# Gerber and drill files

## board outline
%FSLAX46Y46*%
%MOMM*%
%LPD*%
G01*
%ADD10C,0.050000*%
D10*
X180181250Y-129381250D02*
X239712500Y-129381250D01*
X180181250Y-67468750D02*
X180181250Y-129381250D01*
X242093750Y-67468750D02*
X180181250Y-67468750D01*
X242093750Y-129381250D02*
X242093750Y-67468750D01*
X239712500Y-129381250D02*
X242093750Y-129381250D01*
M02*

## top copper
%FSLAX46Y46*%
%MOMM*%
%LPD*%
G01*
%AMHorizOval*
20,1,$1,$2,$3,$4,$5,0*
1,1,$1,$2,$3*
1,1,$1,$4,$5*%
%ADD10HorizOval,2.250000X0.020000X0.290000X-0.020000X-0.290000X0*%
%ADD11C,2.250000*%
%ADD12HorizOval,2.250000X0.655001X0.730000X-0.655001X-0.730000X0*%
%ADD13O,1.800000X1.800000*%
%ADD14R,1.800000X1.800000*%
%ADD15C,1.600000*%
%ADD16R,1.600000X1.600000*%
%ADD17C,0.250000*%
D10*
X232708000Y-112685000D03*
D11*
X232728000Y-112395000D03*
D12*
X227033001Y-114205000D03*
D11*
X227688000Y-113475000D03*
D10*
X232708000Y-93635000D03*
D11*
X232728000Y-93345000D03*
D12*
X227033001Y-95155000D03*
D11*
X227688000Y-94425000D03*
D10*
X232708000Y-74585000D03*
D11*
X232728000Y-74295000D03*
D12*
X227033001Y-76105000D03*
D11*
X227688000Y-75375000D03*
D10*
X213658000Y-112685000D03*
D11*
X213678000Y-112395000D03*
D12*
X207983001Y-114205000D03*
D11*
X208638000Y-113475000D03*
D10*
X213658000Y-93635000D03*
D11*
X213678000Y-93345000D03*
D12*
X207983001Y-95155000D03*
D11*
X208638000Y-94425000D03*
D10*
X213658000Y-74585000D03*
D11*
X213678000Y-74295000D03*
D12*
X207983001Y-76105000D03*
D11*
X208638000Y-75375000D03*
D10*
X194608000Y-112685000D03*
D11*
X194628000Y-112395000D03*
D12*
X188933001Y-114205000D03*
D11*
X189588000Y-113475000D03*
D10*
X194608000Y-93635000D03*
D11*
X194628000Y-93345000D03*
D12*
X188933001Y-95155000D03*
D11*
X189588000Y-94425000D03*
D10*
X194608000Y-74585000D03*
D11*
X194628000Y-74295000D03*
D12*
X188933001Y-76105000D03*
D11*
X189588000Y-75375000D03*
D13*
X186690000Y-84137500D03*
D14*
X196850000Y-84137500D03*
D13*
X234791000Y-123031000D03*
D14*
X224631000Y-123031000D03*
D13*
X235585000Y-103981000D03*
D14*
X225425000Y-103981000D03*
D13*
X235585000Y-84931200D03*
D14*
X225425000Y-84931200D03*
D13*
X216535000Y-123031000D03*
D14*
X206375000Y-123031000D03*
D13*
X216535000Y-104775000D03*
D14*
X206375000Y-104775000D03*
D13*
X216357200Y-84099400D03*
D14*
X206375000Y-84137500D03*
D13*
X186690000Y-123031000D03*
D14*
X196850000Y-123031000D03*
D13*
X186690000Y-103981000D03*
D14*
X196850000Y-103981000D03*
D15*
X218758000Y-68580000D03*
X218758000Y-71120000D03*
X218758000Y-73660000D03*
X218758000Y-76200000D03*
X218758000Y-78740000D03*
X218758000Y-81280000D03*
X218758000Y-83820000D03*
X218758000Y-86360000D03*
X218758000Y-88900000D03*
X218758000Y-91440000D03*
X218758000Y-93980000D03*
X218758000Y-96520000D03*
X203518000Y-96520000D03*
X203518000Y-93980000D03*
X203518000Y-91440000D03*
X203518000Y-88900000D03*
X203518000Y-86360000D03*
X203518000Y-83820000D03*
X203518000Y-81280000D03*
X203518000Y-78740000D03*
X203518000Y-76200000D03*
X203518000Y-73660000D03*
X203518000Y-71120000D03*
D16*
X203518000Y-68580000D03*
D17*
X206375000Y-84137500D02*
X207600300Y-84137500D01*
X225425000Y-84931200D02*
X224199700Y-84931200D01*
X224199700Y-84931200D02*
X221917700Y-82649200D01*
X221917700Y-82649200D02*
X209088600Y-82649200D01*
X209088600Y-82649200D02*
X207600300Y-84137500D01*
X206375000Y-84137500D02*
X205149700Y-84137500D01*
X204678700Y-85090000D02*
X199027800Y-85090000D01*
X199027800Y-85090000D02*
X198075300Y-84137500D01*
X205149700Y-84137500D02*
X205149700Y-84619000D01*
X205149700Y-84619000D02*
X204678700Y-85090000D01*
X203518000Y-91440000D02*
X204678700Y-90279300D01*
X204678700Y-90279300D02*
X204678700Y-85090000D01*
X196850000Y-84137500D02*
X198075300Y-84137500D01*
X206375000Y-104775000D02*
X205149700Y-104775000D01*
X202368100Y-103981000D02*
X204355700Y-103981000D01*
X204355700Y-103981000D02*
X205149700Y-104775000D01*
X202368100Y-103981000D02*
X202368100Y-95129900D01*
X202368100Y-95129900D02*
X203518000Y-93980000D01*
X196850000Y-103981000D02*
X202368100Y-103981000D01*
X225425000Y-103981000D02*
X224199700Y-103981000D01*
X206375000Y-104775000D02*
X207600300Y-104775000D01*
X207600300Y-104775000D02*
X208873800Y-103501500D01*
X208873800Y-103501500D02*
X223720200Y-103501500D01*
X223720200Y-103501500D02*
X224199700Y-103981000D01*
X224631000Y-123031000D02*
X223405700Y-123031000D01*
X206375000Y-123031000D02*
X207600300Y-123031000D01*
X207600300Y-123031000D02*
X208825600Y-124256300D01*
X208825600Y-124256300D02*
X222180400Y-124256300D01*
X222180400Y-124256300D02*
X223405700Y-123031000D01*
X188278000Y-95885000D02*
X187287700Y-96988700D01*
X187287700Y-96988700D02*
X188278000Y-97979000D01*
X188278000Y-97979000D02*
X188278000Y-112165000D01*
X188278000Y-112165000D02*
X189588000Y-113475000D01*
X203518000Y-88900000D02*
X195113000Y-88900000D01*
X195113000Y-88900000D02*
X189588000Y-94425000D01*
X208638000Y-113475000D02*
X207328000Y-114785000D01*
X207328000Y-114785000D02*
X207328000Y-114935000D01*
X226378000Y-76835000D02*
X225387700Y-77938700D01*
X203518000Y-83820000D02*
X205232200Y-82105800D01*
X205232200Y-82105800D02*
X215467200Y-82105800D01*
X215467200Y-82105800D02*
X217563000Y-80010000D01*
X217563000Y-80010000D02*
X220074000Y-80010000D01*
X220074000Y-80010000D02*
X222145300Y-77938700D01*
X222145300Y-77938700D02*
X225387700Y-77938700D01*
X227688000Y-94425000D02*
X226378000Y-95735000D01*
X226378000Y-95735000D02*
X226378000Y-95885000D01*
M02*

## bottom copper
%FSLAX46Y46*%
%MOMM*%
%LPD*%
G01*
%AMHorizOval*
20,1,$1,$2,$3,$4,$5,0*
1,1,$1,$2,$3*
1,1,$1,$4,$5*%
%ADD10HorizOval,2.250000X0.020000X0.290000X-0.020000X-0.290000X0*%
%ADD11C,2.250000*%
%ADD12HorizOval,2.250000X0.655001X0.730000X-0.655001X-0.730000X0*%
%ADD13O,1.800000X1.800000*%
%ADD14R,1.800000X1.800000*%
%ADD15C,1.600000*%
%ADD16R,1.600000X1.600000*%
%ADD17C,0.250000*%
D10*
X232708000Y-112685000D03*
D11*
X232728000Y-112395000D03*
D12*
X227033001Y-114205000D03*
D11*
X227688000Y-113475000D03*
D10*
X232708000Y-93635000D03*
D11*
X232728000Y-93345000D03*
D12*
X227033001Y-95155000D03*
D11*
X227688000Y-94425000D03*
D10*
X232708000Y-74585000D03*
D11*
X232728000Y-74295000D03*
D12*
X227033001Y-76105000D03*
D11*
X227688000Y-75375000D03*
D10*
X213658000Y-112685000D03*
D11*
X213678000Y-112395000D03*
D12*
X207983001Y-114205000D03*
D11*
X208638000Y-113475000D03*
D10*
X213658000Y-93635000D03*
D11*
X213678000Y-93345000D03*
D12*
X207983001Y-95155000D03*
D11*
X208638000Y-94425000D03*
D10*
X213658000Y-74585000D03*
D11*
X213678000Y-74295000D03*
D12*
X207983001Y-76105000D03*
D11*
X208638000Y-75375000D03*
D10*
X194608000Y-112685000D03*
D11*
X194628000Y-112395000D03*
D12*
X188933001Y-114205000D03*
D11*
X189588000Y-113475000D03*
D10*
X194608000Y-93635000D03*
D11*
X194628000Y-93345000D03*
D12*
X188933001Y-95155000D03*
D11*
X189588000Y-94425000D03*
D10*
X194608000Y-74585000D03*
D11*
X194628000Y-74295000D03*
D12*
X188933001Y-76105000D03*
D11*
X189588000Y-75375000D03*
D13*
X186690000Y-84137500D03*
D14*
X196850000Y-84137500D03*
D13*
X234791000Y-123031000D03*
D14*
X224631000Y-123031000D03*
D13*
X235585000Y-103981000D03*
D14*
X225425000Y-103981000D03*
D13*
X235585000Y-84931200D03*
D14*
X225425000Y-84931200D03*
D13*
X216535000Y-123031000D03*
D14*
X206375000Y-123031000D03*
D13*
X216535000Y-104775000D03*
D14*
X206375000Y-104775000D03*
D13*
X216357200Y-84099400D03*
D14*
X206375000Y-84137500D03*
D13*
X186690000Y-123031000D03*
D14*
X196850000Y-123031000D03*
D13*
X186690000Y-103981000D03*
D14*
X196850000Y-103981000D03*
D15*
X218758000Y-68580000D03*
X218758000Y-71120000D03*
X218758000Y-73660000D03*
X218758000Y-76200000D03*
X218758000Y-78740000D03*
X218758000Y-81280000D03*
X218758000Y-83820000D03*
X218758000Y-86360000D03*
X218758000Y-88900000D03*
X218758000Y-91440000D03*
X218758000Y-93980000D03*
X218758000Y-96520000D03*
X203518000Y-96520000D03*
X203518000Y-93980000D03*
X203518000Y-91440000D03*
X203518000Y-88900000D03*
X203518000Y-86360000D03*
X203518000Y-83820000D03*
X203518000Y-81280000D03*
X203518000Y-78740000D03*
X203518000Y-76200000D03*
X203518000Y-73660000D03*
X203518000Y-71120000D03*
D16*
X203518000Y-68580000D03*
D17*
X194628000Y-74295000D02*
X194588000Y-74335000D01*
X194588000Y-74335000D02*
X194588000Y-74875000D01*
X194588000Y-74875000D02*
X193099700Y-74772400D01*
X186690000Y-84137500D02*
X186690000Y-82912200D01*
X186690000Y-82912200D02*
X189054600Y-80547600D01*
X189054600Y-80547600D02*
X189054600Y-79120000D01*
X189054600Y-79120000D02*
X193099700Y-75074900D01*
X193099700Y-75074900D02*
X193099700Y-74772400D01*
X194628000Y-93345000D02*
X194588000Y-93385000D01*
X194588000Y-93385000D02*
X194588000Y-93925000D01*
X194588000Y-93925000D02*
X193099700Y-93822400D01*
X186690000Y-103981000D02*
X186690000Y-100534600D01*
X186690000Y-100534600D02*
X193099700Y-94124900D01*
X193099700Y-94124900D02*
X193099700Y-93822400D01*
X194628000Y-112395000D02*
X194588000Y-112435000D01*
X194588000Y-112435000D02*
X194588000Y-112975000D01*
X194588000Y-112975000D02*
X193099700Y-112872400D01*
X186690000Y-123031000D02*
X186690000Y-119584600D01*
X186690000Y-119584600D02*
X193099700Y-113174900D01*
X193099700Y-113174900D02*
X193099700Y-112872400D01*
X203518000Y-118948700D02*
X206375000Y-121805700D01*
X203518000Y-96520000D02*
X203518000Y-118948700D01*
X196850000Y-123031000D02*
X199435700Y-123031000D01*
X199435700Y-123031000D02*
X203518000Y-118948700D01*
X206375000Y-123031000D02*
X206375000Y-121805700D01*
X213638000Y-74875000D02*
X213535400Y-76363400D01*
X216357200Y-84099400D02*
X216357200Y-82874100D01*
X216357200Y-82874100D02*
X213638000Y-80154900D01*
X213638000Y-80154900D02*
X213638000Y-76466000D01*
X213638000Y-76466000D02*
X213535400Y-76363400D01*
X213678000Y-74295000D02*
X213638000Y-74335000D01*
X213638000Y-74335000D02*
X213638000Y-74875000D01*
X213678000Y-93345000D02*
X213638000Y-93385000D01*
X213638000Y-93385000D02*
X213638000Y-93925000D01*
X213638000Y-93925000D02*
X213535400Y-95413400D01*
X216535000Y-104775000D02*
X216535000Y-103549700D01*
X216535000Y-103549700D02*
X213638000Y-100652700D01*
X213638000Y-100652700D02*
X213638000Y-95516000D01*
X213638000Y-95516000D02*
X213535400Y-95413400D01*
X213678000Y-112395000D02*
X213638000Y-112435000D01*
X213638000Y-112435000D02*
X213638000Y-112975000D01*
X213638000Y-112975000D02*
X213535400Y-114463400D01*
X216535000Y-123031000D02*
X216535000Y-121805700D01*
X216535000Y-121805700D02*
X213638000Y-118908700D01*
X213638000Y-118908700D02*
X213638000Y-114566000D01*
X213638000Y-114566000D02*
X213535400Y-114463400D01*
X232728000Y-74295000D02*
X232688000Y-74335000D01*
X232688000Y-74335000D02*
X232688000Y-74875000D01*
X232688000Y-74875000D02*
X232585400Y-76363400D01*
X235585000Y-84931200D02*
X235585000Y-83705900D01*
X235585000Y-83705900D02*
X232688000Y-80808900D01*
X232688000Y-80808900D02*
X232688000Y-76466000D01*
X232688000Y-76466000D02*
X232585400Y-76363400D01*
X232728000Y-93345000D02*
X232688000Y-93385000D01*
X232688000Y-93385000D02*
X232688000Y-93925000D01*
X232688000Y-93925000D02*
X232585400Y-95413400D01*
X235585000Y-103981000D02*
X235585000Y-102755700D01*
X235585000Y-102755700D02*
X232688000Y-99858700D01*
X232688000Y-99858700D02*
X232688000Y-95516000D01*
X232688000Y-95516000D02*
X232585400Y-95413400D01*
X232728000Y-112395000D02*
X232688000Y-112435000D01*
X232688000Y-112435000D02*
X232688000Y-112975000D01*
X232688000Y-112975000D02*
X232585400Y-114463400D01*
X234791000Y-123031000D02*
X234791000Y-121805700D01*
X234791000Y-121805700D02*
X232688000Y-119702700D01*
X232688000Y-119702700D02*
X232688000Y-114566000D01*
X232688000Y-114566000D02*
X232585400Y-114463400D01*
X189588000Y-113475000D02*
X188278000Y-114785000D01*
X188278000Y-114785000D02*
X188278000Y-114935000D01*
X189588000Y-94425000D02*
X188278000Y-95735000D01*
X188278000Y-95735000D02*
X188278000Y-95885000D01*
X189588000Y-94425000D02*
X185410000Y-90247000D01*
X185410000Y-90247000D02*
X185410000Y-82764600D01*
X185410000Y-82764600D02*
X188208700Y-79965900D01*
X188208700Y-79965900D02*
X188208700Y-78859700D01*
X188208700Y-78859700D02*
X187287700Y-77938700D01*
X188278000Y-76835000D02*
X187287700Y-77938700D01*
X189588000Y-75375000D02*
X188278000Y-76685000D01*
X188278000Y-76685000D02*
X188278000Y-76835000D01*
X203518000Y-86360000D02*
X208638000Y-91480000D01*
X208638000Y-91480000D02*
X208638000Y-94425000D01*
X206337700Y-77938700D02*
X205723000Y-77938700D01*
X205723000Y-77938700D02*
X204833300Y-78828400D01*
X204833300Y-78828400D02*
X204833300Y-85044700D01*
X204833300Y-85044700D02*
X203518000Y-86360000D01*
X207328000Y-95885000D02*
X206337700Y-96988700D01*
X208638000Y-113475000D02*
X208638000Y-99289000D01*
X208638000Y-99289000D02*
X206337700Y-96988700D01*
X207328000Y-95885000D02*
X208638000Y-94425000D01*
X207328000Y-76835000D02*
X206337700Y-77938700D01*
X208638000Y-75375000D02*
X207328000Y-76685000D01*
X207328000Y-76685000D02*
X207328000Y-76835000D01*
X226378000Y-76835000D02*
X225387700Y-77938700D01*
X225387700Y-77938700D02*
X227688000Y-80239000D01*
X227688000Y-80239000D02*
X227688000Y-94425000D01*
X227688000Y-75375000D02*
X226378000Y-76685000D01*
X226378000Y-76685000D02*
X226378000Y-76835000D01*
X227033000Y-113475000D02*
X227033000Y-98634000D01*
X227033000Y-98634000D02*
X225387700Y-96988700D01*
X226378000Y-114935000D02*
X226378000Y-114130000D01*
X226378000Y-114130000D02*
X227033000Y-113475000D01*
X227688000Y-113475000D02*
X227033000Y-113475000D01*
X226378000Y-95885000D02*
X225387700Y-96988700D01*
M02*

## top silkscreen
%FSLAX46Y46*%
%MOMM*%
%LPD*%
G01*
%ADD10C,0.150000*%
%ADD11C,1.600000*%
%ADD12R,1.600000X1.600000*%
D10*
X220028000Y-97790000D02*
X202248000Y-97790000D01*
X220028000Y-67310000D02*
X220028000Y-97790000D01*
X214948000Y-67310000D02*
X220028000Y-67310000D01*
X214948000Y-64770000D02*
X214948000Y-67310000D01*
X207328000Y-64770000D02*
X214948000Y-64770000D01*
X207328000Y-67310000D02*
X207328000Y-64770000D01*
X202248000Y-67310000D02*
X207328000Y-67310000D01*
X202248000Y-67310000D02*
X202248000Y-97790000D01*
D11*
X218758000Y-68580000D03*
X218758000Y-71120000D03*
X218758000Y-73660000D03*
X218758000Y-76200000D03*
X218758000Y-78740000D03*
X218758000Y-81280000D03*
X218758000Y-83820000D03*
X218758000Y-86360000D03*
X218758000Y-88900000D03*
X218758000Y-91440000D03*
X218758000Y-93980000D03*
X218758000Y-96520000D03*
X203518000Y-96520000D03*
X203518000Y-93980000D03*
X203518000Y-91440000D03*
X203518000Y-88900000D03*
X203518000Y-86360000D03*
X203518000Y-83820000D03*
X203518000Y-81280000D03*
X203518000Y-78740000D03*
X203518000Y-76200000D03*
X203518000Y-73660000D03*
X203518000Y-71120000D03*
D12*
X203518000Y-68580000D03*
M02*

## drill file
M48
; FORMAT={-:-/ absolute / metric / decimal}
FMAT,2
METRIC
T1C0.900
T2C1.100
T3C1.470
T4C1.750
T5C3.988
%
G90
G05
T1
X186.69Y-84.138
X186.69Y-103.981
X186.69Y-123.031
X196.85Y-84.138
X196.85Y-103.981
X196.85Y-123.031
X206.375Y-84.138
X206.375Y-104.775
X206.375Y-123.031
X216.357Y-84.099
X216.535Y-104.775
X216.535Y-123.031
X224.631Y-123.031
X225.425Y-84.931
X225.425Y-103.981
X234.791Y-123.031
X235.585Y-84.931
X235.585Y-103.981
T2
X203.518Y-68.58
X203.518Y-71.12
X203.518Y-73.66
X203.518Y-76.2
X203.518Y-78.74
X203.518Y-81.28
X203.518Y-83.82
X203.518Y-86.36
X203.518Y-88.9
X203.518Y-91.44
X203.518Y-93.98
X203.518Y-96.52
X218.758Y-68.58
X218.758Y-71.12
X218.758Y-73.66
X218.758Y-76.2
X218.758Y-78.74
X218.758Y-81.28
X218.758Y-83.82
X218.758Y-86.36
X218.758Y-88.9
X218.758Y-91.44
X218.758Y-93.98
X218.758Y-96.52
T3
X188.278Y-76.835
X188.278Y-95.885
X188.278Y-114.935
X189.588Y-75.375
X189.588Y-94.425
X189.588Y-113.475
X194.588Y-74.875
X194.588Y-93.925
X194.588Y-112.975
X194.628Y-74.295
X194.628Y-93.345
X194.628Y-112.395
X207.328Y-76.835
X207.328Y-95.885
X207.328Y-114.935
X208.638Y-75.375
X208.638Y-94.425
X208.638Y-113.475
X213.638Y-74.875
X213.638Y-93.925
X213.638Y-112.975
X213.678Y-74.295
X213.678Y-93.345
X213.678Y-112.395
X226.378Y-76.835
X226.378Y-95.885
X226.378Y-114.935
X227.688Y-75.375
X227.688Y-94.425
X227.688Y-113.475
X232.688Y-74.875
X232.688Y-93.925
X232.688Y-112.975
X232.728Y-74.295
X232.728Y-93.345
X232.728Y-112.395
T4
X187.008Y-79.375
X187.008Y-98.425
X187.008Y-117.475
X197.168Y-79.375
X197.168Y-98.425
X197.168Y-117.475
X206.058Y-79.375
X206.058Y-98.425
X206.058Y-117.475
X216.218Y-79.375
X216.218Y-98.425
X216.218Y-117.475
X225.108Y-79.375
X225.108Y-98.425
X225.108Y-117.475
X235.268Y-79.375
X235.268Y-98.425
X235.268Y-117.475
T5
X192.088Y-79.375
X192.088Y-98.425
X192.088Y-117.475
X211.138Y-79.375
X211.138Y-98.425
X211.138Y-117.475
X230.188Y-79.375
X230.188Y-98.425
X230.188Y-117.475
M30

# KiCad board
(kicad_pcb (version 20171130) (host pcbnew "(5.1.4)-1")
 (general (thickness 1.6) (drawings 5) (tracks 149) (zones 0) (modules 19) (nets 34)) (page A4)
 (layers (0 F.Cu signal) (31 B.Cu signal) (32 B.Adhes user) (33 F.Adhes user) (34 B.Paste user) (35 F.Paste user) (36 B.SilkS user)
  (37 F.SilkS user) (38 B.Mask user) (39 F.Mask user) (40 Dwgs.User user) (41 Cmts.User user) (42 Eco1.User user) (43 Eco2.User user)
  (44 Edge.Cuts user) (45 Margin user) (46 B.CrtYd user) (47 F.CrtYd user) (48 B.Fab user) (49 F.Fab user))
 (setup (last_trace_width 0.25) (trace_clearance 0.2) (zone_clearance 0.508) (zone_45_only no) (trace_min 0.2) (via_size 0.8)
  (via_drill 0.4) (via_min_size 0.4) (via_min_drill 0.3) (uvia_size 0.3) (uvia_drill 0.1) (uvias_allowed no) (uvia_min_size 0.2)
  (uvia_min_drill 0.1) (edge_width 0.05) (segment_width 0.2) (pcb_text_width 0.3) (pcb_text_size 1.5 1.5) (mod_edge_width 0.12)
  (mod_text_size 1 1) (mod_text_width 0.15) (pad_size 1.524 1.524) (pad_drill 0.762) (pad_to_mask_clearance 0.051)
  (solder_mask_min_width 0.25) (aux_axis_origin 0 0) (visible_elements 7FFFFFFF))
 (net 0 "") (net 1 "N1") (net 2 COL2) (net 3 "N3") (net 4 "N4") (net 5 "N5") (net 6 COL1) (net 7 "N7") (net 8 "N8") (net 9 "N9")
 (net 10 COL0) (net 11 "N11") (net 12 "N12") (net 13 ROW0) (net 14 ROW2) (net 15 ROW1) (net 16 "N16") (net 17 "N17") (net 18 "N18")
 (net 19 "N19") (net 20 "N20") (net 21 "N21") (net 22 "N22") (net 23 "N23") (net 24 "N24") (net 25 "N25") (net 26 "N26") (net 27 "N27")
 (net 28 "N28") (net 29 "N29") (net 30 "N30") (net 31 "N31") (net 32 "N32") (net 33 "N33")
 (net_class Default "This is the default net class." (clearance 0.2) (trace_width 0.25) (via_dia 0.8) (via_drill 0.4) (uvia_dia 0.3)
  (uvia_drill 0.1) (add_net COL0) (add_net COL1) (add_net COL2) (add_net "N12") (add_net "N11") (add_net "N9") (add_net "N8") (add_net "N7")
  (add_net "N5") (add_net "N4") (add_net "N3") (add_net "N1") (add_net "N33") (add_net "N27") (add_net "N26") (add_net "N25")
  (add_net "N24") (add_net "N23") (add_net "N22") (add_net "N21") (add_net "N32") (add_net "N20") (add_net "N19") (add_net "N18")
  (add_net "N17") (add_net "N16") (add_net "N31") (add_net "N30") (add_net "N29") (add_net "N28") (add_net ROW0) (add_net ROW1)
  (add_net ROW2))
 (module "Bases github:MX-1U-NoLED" (layer F.Cu) (at 230.188 117.475)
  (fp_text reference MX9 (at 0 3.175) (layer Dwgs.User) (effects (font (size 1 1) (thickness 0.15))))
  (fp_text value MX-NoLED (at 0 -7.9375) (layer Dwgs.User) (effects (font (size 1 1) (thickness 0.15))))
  (pad 2 thru_hole oval (at 2.5 -4.5 86.0548) (size 2.831378 2.25) (drill 1.47 (offset 0.290689 0)) (layers *.Cu B.Mask) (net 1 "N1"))
  (pad 2 thru_hole circle (at 2.54 -5.08) (size 2.25 2.25) (drill 1.47) (layers *.Cu B.Mask) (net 1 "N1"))
  (pad 1 thru_hole oval (at -3.81 -2.54 48.0996) (size 4.211556 2.25) (drill 1.47 (offset 0.980778 0)) (layers *.Cu B.Mask) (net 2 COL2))
  (pad "" np_thru_hole circle (at 0 0) (size 3.9878 3.9878) (drill 3.9878) (layers *.Cu *.Mask))
  (pad 1 thru_hole circle (at -2.5 -4) (size 2.25 2.25) (drill 1.47) (layers *.Cu B.Mask) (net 2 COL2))
  (pad "" np_thru_hole circle (at -5.08 0 48.0996) (size 1.75 1.75) (drill 1.75) (layers *.Cu *.Mask))
  (pad "" np_thru_hole circle (at 5.08 0 48.0996) (size 1.75 1.75) (drill 1.75) (layers *.Cu *.Mask)))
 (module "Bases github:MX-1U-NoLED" (layer F.Cu) (at 230.188 98.425)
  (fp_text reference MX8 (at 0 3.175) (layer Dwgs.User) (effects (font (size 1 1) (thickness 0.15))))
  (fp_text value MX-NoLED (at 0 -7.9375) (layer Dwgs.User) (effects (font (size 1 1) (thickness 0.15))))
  (pad 2 thru_hole oval (at 2.5 -4.5 86.0548) (size 2.831378 2.25) (drill 1.47 (offset 0.290689 0)) (layers *.Cu B.Mask) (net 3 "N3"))
  (pad 2 thru_hole circle (at 2.54 -5.08) (size 2.25 2.25) (drill 1.47) (layers *.Cu B.Mask) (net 3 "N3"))
  (pad 1 thru_hole oval (at -3.81 -2.54 48.0996) (size 4.211556 2.25) (drill 1.47 (offset 0.980778 0)) (layers *.Cu B.Mask) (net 2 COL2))
  (pad "" np_thru_hole circle (at 0 0) (size 3.9878 3.9878) (drill 3.9878) (layers *.Cu *.Mask))
  (pad 1 thru_hole circle (at -2.5 -4) (size 2.25 2.25) (drill 1.47) (layers *.Cu B.Mask) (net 2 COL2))
  (pad "" np_thru_hole circle (at -5.08 0 48.0996) (size 1.75 1.75) (drill 1.75) (layers *.Cu *.Mask))
  (pad "" np_thru_hole circle (at 5.08 0 48.0996) (size 1.75 1.75) (drill 1.75) (layers *.Cu *.Mask)))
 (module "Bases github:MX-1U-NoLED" (layer F.Cu) (at 230.188 79.375)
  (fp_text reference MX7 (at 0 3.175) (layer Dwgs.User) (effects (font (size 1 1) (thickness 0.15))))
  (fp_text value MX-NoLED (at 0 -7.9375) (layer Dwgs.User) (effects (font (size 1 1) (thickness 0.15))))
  (pad 2 thru_hole oval (at 2.5 -4.5 86.0548) (size 2.831378 2.25) (drill 1.47 (offset 0.290689 0)) (layers *.Cu B.Mask) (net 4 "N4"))
  (pad 2 thru_hole circle (at 2.54 -5.08) (size 2.25 2.25) (drill 1.47) (layers *.Cu B.Mask) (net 4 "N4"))
  (pad 1 thru_hole oval (at -3.81 -2.54 48.0996) (size 4.211556 2.25) (drill 1.47 (offset 0.980778 0)) (layers *.Cu B.Mask) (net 2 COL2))
  (pad "" np_thru_hole circle (at 0 0) (size 3.9878 3.9878) (drill 3.9878) (layers *.Cu *.Mask))
  (pad 1 thru_hole circle (at -2.5 -4) (size 2.25 2.25) (drill 1.47) (layers *.Cu B.Mask) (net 2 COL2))
  (pad "" np_thru_hole circle (at -5.08 0 48.0996) (size 1.75 1.75) (drill 1.75) (layers *.Cu *.Mask))
  (pad "" np_thru_hole circle (at 5.08 0 48.0996) (size 1.75 1.75) (drill 1.75) (layers *.Cu *.Mask)))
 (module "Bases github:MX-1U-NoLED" (layer F.Cu) (at 211.138 117.475)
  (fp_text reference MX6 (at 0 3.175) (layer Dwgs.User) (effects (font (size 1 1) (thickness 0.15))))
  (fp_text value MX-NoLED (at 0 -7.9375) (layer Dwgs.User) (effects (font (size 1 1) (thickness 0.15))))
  (pad 2 thru_hole oval (at 2.5 -4.5 86.0548) (size 2.831378 2.25) (drill 1.47 (offset 0.290689 0)) (layers *.Cu B.Mask) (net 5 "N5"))
  (pad 2 thru_hole circle (at 2.54 -5.08) (size 2.25 2.25) (drill 1.47) (layers *.Cu B.Mask) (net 5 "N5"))
  (pad 1 thru_hole oval (at -3.81 -2.54 48.0996) (size 4.211556 2.25) (drill 1.47 (offset 0.980778 0)) (layers *.Cu B.Mask) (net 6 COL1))
  (pad "" np_thru_hole circle (at 0 0) (size 3.9878 3.9878) (drill 3.9878) (layers *.Cu *.Mask))
  (pad 1 thru_hole circle (at -2.5 -4) (size 2.25 2.25) (drill 1.47) (layers *.Cu B.Mask) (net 6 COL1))
  (pad "" np_thru_hole circle (at -5.08 0 48.0996) (size 1.75 1.75) (drill 1.75) (layers *.Cu *.Mask))
  (pad "" np_thru_hole circle (at 5.08 0 48.0996) (size 1.75 1.75) (drill 1.75) (layers *.Cu *.Mask)))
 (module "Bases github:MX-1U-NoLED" (layer F.Cu) (at 211.138 98.425)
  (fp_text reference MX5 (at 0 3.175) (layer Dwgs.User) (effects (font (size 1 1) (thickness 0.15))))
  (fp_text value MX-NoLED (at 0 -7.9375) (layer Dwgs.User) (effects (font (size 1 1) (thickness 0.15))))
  (pad 2 thru_hole oval (at 2.5 -4.5 86.0548) (size 2.831378 2.25) (drill 1.47 (offset 0.290689 0)) (layers *.Cu B.Mask) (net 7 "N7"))
  (pad 2 thru_hole circle (at 2.54 -5.08) (size 2.25 2.25) (drill 1.47) (layers *.Cu B.Mask) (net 7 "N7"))
  (pad 1 thru_hole oval (at -3.81 -2.54 48.0996) (size 4.211556 2.25) (drill 1.47 (offset 0.980778 0)) (layers *.Cu B.Mask) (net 6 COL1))
  (pad "" np_thru_hole circle (at 0 0) (size 3.9878 3.9878) (drill 3.9878) (layers *.Cu *.Mask))
  (pad 1 thru_hole circle (at -2.5 -4) (size 2.25 2.25) (drill 1.47) (layers *.Cu B.Mask) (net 6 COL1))
  (pad "" np_thru_hole circle (at -5.08 0 48.0996) (size 1.75 1.75) (drill 1.75) (layers *.Cu *.Mask))
  (pad "" np_thru_hole circle (at 5.08 0 48.0996) (size 1.75 1.75) (drill 1.75) (layers *.Cu *.Mask)))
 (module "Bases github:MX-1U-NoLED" (layer F.Cu) (at 211.138 79.375)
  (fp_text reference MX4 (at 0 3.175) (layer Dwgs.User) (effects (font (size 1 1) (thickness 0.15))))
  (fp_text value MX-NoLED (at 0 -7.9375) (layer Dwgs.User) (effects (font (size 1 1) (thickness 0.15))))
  (pad 2 thru_hole oval (at 2.5 -4.5 86.0548) (size 2.831378 2.25) (drill 1.47 (offset 0.290689 0)) (layers *.Cu B.Mask) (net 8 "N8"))
  (pad 2 thru_hole circle (at 2.54 -5.08) (size 2.25 2.25) (drill 1.47) (layers *.Cu B.Mask) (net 8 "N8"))
  (pad 1 thru_hole oval (at -3.81 -2.54 48.0996) (size 4.211556 2.25) (drill 1.47 (offset 0.980778 0)) (layers *.Cu B.Mask) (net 6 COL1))
  (pad "" np_thru_hole circle (at 0 0) (size 3.9878 3.9878) (drill 3.9878) (layers *.Cu *.Mask))
  (pad 1 thru_hole circle (at -2.5 -4) (size 2.25 2.25) (drill 1.47) (layers *.Cu B.Mask) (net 6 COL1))
  (pad "" np_thru_hole circle (at -5.08 0 48.0996) (size 1.75 1.75) (drill 1.75) (layers *.Cu *.Mask))
  (pad "" np_thru_hole circle (at 5.08 0 48.0996) (size 1.75 1.75) (drill 1.75) (layers *.Cu *.Mask)))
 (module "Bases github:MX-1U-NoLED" (layer F.Cu) (at 192.088 117.475)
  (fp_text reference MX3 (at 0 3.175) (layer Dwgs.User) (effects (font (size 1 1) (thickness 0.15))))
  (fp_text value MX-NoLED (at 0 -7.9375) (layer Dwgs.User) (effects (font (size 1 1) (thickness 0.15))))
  (pad 2 thru_hole oval (at 2.5 -4.5 86.0548) (size 2.831378 2.25) (drill 1.47 (offset 0.290689 0)) (layers *.Cu B.Mask) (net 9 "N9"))
  (pad 2 thru_hole circle (at 2.54 -5.08) (size 2.25 2.25) (drill 1.47) (layers *.Cu B.Mask) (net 9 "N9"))
  (pad 1 thru_hole oval (at -3.81 -2.54 48.0996) (size 4.211556 2.25) (drill 1.47 (offset 0.980778 0)) (layers *.Cu B.Mask) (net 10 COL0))
  (pad "" np_thru_hole circle (at 0 0) (size 3.9878 3.9878) (drill 3.9878) (layers *.Cu *.Mask))
  (pad 1 thru_hole circle (at -2.5 -4) (size 2.25 2.25) (drill 1.47) (layers *.Cu B.Mask) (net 10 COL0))
  (pad "" np_thru_hole circle (at -5.08 0 48.0996) (size 1.75 1.75) (drill 1.75) (layers *.Cu *.Mask))
  (pad "" np_thru_hole circle (at 5.08 0 48.0996) (size 1.75 1.75) (drill 1.75) (layers *.Cu *.Mask)))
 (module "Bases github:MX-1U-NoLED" (layer F.Cu) (at 192.088 98.425)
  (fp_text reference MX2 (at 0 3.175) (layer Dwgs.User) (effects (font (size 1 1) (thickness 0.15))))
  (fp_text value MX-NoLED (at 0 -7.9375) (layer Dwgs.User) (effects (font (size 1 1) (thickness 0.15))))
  (pad 2 thru_hole oval (at 2.5 -4.5 86.0548) (size 2.831378 2.25) (drill 1.47 (offset 0.290689 0)) (layers *.Cu B.Mask) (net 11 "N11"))
  (pad 2 thru_hole circle (at 2.54 -5.08) (size 2.25 2.25) (drill 1.47) (layers *.Cu B.Mask) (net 11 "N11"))
  (pad 1 thru_hole oval (at -3.81 -2.54 48.0996) (size 4.211556 2.25) (drill 1.47 (offset 0.980778 0)) (layers *.Cu B.Mask) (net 10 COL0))
  (pad "" np_thru_hole circle (at 0 0) (size 3.9878 3.9878) (drill 3.9878) (layers *.Cu *.Mask))
  (pad 1 thru_hole circle (at -2.5 -4) (size 2.25 2.25) (drill 1.47) (layers *.Cu B.Mask) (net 10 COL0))
  (pad "" np_thru_hole circle (at -5.08 0 48.0996) (size 1.75 1.75) (drill 1.75) (layers *.Cu *.Mask))
  (pad "" np_thru_hole circle (at 5.08 0 48.0996) (size 1.75 1.75) (drill 1.75) (layers *.Cu *.Mask)))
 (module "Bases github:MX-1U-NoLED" (layer F.Cu) (at 192.088 79.375)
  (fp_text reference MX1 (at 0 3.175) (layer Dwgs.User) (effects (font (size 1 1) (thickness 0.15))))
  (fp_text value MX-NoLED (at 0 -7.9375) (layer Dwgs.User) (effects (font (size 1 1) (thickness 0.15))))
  (pad 2 thru_hole oval (at 2.5 -4.5 86.0548) (size 2.831378 2.25) (drill 1.47 (offset 0.290689 0)) (layers *.Cu B.Mask) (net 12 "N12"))
  (pad 2 thru_hole circle (at 2.54 -5.08) (size 2.25 2.25) (drill 1.47) (layers *.Cu B.Mask) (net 12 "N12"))
  (pad 1 thru_hole oval (at -3.81 -2.54 48.0996) (size 4.211556 2.25) (drill 1.47 (offset 0.980778 0)) (layers *.Cu B.Mask) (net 10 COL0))
  (pad "" np_thru_hole circle (at 0 0) (size 3.9878 3.9878) (drill 3.9878) (layers *.Cu *.Mask))
  (pad 1 thru_hole circle (at -2.5 -4) (size 2.25 2.25) (drill 1.47) (layers *.Cu B.Mask) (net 10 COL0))
  (pad "" np_thru_hole circle (at -5.08 0 48.0996) (size 1.75 1.75) (drill 1.75) (layers *.Cu *.Mask))
  (pad "" np_thru_hole circle (at 5.08 0 48.0996) (size 1.75 1.75) (drill 1.75) (layers *.Cu *.Mask)))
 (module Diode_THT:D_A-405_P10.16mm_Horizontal (layer B.Cu) (at 196.85 84.1375 180)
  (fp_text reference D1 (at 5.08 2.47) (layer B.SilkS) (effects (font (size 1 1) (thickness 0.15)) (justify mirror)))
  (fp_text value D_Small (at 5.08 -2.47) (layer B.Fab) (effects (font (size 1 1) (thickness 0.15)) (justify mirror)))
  (pad 2 thru_hole oval (at 10.16 0 180) (size 1.8 1.8) (drill 0.9) (layers *.Cu *.Mask) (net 12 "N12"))
  (pad 1 thru_hole rect (at 0 0 180) (size 1.8 1.8) (drill 0.9) (layers *.Cu *.Mask) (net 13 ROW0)))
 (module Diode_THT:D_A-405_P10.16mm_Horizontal (layer B.Cu) (at 224.631 123.031)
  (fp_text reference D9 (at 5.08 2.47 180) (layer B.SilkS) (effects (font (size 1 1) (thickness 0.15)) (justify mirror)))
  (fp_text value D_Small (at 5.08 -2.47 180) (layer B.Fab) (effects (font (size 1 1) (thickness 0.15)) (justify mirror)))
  (pad 2 thru_hole oval (at 10.16 0) (size 1.8 1.8) (drill 0.9) (layers *.Cu *.Mask) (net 1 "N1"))
  (pad 1 thru_hole rect (at 0 0) (size 1.8 1.8) (drill 0.9) (layers *.Cu *.Mask) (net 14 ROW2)))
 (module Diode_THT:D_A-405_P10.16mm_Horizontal (layer B.Cu) (at 225.425 103.981)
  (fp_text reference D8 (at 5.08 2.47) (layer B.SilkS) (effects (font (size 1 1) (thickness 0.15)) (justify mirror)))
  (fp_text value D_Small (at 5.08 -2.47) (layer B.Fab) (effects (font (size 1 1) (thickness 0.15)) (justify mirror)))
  (pad 2 thru_hole oval (at 10.16 0) (size 1.8 1.8) (drill 0.9) (layers *.Cu *.Mask) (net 3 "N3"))
  (pad 1 thru_hole rect (at 0 0) (size 1.8 1.8) (drill 0.9) (layers *.Cu *.Mask) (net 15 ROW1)))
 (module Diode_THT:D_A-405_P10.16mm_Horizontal (layer B.Cu) (at 225.425 84.9312)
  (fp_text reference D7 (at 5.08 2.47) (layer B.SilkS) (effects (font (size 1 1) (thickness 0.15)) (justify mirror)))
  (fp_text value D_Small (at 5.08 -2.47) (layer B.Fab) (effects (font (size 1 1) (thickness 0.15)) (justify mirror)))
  (pad 2 thru_hole oval (at 10.16 0) (size 1.8 1.8) (drill 0.9) (layers *.Cu *.Mask) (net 4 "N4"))
  (pad 1 thru_hole rect (at 0 0) (size 1.8 1.8) (drill 0.9) (layers *.Cu *.Mask) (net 13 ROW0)))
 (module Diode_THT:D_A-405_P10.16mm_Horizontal (layer B.Cu) (at 206.375 123.031)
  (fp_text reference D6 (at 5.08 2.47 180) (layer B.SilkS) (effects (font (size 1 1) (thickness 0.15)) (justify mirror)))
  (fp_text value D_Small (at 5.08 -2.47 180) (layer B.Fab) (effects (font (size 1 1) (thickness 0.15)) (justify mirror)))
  (pad 2 thru_hole oval (at 10.16 0) (size 1.8 1.8) (drill 0.9) (layers *.Cu *.Mask) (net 5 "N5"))
  (pad 1 thru_hole rect (at 0 0) (size 1.8 1.8) (drill 0.9) (layers *.Cu *.Mask) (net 14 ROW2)))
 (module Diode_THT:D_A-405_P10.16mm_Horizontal (layer B.Cu) (at 206.375 104.775)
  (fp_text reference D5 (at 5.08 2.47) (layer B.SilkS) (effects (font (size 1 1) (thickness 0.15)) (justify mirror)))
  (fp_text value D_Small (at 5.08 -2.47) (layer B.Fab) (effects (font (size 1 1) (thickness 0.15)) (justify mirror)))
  (pad 2 thru_hole oval (at 10.16 0) (size 1.8 1.8) (drill 0.9) (layers *.Cu *.Mask) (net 7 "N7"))
  (pad 1 thru_hole rect (at 0 0) (size 1.8 1.8) (drill 0.9) (layers *.Cu *.Mask) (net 15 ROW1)))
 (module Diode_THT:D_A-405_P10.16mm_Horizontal (layer B.Cu) (at 206.375 84.1375)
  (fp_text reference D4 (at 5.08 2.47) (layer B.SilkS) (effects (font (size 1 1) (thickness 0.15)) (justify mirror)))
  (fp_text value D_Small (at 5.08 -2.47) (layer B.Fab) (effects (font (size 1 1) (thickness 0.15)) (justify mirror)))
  (pad 2 thru_hole oval (at 9.9822 -0.0381) (size 1.8 1.8) (drill 0.9) (layers *.Cu *.Mask) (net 8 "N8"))
  (pad 1 thru_hole rect (at 0 0) (size 1.8 1.8) (drill 0.9) (layers *.Cu *.Mask) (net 13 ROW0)))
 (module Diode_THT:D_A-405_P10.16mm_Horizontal (layer B.Cu) (at 196.85 123.031 180)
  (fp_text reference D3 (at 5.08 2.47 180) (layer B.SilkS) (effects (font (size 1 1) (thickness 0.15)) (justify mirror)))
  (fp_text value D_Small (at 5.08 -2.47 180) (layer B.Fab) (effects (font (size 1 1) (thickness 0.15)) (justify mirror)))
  (pad 2 thru_hole oval (at 10.16 0 180) (size 1.8 1.8) (drill 0.9) (layers *.Cu *.Mask) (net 9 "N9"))
  (pad 1 thru_hole rect (at 0 0 180) (size 1.8 1.8) (drill 0.9) (layers *.Cu *.Mask) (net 14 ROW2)))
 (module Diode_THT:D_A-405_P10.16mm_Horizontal (layer B.Cu) (at 196.85 103.981 180)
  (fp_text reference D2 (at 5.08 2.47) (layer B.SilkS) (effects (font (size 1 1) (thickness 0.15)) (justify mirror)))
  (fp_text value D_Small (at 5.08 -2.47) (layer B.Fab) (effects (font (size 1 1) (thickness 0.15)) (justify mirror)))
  (pad 2 thru_hole oval (at 10.16 0 180) (size 1.8 1.8) (drill 0.9) (layers *.Cu *.Mask) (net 11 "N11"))
  (pad 1 thru_hole rect (at 0 0 180) (size 1.8 1.8) (drill 0.9) (layers *.Cu *.Mask) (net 15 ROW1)))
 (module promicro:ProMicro (layer F.Cu) (at 211.138 82.55 270)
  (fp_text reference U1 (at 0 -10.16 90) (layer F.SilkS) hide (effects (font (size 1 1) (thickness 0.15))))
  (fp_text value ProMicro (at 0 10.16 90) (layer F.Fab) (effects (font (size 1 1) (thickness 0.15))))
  (fp_line (start 15.24 -8.89) (end 15.24 8.89) (layer F.SilkS) (width 0.15))
  (fp_line (start -15.24 -8.89) (end 15.24 -8.89) (layer F.SilkS) (width 0.15))
  (fp_line (start -15.24 -3.81) (end -15.24 -8.89) (layer F.SilkS) (width 0.15))
  (fp_line (start -17.78 -3.81) (end -15.24 -3.81) (layer F.SilkS) (width 0.15))
  (fp_line (start -17.78 3.81) (end -17.78 -3.81) (layer F.SilkS) (width 0.15))
  (fp_line (start -15.24 3.81) (end -17.78 3.81) (layer F.SilkS) (width 0.15))
  (fp_line (start -15.24 8.89) (end -15.24 3.81) (layer F.SilkS) (width 0.15))
  (fp_line (start -15.24 8.89) (end 15.24 8.89) (layer F.SilkS) (width 0.15))
  (pad 24 thru_hole circle (at -13.97 -7.62 270) (size 1.6 1.6) (drill 1.1) (layers *.Cu *.Mask F.SilkS) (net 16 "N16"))
  (pad 23 thru_hole circle (at -11.43 -7.62 270) (size 1.6 1.6) (drill 1.1) (layers *.Cu *.Mask F.SilkS) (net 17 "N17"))
  (pad 22 thru_hole circle (at -8.89 -7.62 270) (size 1.6 1.6) (drill 1.1) (layers *.Cu *.Mask F.SilkS) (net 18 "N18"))
  (pad 21 thru_hole circle (at -6.35 -7.62 270) (size 1.6 1.6) (drill 1.1) (layers *.Cu *.Mask F.SilkS) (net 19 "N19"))
  (pad 20 thru_hole circle (at -3.81 -7.62 270) (size 1.6 1.6) (drill 1.1) (layers *.Cu *.Mask F.SilkS) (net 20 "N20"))
  (pad 19 thru_hole circle (at -1.27 -7.62 270) (size 1.6 1.6) (drill 1.1) (layers *.Cu *.Mask F.SilkS) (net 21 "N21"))
  (pad 18 thru_hole circle (at 1.27 -7.62 270) (size 1.6 1.6) (drill 1.1) (layers *.Cu *.Mask F.SilkS) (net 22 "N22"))
  (pad 17 thru_hole circle (at 3.81 -7.62 270) (size 1.6 1.6) (drill 1.1) (layers *.Cu *.Mask F.SilkS) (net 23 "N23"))
  (pad 16 thru_hole circle (at 6.35 -7.62 270) (size 1.6 1.6) (drill 1.1) (layers *.Cu *.Mask F.SilkS) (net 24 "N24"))
  (pad 15 thru_hole circle (at 8.89 -7.62 270) (size 1.6 1.6) (drill 1.1) (layers *.Cu *.Mask F.SilkS) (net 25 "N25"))
  (pad 14 thru_hole circle (at 11.43 -7.62 270) (size 1.6 1.6) (drill 1.1) (layers *.Cu *.Mask F.SilkS) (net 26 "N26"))
  (pad 13 thru_hole circle (at 13.97 -7.62 270) (size 1.6 1.6) (drill 1.1) (layers *.Cu *.Mask F.SilkS) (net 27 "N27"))
  (pad 12 thru_hole circle (at 13.97 7.62 270) (size 1.6 1.6) (drill 1.1) (layers *.Cu *.Mask F.SilkS) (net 14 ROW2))
  (pad 11 thru_hole circle (at 11.43 7.62 270) (size 1.6 1.6) (drill 1.1) (layers *.Cu *.Mask F.SilkS) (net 15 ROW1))
  (pad 10 thru_hole circle (at 8.89 7.62 270) (size 1.6 1.6) (drill 1.1) (layers *.Cu *.Mask F.SilkS) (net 13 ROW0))
  (pad 9 thru_hole circle (at 6.35 7.62 270) (size 1.6 1.6) (drill 1.1) (layers *.Cu *.Mask F.SilkS) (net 10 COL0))
  (pad 8 thru_hole circle (at 3.81 7.62 270) (size 1.6 1.6) (drill 1.1) (layers *.Cu *.Mask F.SilkS) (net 6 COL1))
  (pad 7 thru_hole circle (at 1.27 7.62 270) (size 1.6 1.6) (drill 1.1) (layers *.Cu *.Mask F.SilkS) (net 2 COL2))
  (pad 6 thru_hole circle (at -1.27 7.62 270) (size 1.6 1.6) (drill 1.1) (layers *.Cu *.Mask F.SilkS) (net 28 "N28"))
  (pad 5 thru_hole circle (at -3.81 7.62 270) (size 1.6 1.6) (drill 1.1) (layers *.Cu *.Mask F.SilkS) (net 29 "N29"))
  (pad 4 thru_hole circle (at -6.35 7.62 270) (size 1.6 1.6) (drill 1.1) (layers *.Cu *.Mask F.SilkS) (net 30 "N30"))
  (pad 3 thru_hole circle (at -8.89 7.62 270) (size 1.6 1.6) (drill 1.1) (layers *.Cu *.Mask F.SilkS) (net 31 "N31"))
  (pad 2 thru_hole circle (at -11.43 7.62 270) (size 1.6 1.6) (drill 1.1) (layers *.Cu *.Mask F.SilkS) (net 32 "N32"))
  (pad 1 thru_hole rect (at -13.97 7.62 270) (size 1.6 1.6) (drill 1.1) (layers *.Cu *.Mask F.SilkS) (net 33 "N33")))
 (gr_line (start 180.18125 129.38125) (end 239.7125 129.38125) (layer Edge.Cuts) (width 0.05))
 (gr_line (start 180.18125 67.46875) (end 180.18125 129.38125) (layer Edge.Cuts) (width 0.05))
 (gr_line (start 242.09375 67.46875) (end 180.18125 67.46875) (layer Edge.Cuts) (width 0.05))
 (gr_line (start 242.09375 129.38125) (end 242.09375 67.46875) (layer Edge.Cuts) (width 0.05))
 (gr_line (start 239.7125 129.38125) (end 242.09375 129.38125) (layer Edge.Cuts) (width 0.05))
 (segment (start 194.628 74.295) (end 194.588 74.335) (width 0.25) (layer B.Cu) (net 12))
 (segment (start 194.588 74.335) (end 194.588 74.875) (width 0.25) (layer B.Cu) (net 12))
 (segment (start 194.588 74.875) (end 193.0997 74.7724) (width 0.25) (layer B.Cu) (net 12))
 (segment (start 186.69 84.1375) (end 186.69 82.9122) (width 0.25) (layer B.Cu) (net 12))
 (segment (start 186.69 82.9122) (end 189.0546 80.5476) (width 0.25) (layer B.Cu) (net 12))
 (segment (start 189.0546 80.5476) (end 189.0546 79.12) (width 0.25) (layer B.Cu) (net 12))
 (segment (start 189.0546 79.12) (end 193.0997 75.0749) (width 0.25) (layer B.Cu) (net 12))
 (segment (start 193.0997 75.0749) (end 193.0997 74.7724) (width 0.25) (layer B.Cu) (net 12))
 (segment (start 206.375 84.1375) (end 207.6003 84.1375) (width 0.25) (layer F.Cu) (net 13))
 (segment (start 225.425 84.9312) (end 224.1997 84.9312) (width 0.25) (layer F.Cu) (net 13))
 (segment (start 224.1997 84.9312) (end 221.9177 82.6492) (width 0.25) (layer F.Cu) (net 13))
 (segment (start 221.9177 82.6492) (end 209.0886 82.6492) (width 0.25) (layer F.Cu) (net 13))
 (segment (start 209.0886 82.6492) (end 207.6003 84.1375) (width 0.25) (layer F.Cu) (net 13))
 (segment (start 206.375 84.1375) (end 205.1497 84.1375) (width 0.25) (layer F.Cu) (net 13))
 (segment (start 204.6787 85.09) (end 199.0278 85.09) (width 0.25) (layer F.Cu) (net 13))
 (segment (start 199.0278 85.09) (end 198.0753 84.1375) (width 0.25) (layer F.Cu) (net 13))
 (segment (start 205.1497 84.1375) (end 205.1497 84.619) (width 0.25) (layer F.Cu) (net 13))
 (segment (start 205.1497 84.619) (end 204.6787 85.09) (width 0.25) (layer F.Cu) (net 13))
 (segment (start 203.518 91.44) (end 204.6787 90.2793) (width 0.25) (layer F.Cu) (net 13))
 (segment (start 204.6787 90.2793) (end 204.6787 85.09) (width 0.25) (layer F.Cu) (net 13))
 (segment (start 196.85 84.1375) (end 198.0753 84.1375) (width 0.25) (layer F.Cu) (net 13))
 (segment (start 194.628 93.345) (end 194.588 93.385) (width 0.25) (layer B.Cu) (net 11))
 (segment (start 194.588 93.385) (end 194.588 93.925) (width 0.25) (layer B.Cu) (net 11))
 (segment (start 194.588 93.925) (end 193.0997 93.8224) (width 0.25) (layer B.Cu) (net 11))
 (segment (start 186.69 103.981) (end 186.69 100.5346) (width 0.25) (layer B.Cu) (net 11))
 (segment (start 186.69 100.5346) (end 193.0997 94.1249) (width 0.25) (layer B.Cu) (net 11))
 (segment (start 193.0997 94.1249) (end 193.0997 93.8224) (width 0.25) (layer B.Cu) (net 11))
 (segment (start 206.375 104.775) (end 205.1497 104.775) (width 0.25) (layer F.Cu) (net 15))
 (segment (start 202.3681 103.981) (end 204.3557 103.981) (width 0.25) (layer F.Cu) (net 15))
 (segment (start 204.3557 103.981) (end 205.1497 104.775) (width 0.25) (layer F.Cu) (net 15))
 (segment (start 202.3681 103.981) (end 202.3681 95.1299) (width 0.25) (layer F.Cu) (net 15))
 (segment (start 202.3681 95.1299) (end 203.518 93.98) (width 0.25) (layer F.Cu) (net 15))
 (segment (start 196.85 103.981) (end 202.3681 103.981) (width 0.25) (layer F.Cu) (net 15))
 (segment (start 225.425 103.981) (end 224.1997 103.981) (width 0.25) (layer F.Cu) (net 15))
 (segment (start 206.375 104.775) (end 207.6003 104.775) (width 0.25) (layer F.Cu) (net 15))
 (segment (start 207.6003 104.775) (end 208.8738 103.5015) (width 0.25) (layer F.Cu) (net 15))
 (segment (start 208.8738 103.5015) (end 223.7202 103.5015) (width 0.25) (layer F.Cu) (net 15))
 (segment (start 223.7202 103.5015) (end 224.1997 103.981) (width 0.25) (layer F.Cu) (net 15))
 (segment (start 194.628 112.395) (end 194.588 112.435) (width 0.25) (layer B.Cu) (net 9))
 (segment (start 194.588 112.435) (end 194.588 112.975) (width 0.25) (layer B.Cu) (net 9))
 (segment (start 194.588 112.975) (end 193.0997 112.8724) (width 0.25) (layer B.Cu) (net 9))
 (segment (start 186.69 123.031) (end 186.69 119.5846) (width 0.25) (layer B.Cu) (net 9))
 (segment (start 186.69 119.5846) (end 193.0997 113.1749) (width 0.25) (layer B.Cu) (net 9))
 (segment (start 193.0997 113.1749) (end 193.0997 112.8724) (width 0.25) (layer B.Cu) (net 9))
 (segment (start 203.518 118.9487) (end 206.375 121.8057) (width 0.25) (layer B.Cu) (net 14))
 (segment (start 203.518 96.52) (end 203.518 118.9487) (width 0.25) (layer B.Cu) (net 14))
 (segment (start 196.85 123.031) (end 199.4357 123.031) (width 0.25) (layer B.Cu) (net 14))
 (segment (start 199.4357 123.031) (end 203.518 118.9487) (width 0.25) (layer B.Cu) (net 14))
 (segment (start 206.375 123.031) (end 206.375 121.8057) (width 0.25) (layer B.Cu) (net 14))
 (segment (start 224.631 123.031) (end 223.4057 123.031) (width 0.25) (layer F.Cu) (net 14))
 (segment (start 206.375 123.031) (end 207.6003 123.031) (width 0.25) (layer F.Cu) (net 14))
 (segment (start 207.6003 123.031) (end 208.8256 124.2563) (width 0.25) (layer F.Cu) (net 14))
 (segment (start 208.8256 124.2563) (end 222.1804 124.2563) (width 0.25) (layer F.Cu) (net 14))
 (segment (start 222.1804 124.2563) (end 223.4057 123.031) (width 0.25) (layer F.Cu) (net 14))
 (segment (start 213.638 74.875) (end 213.5354 76.3634) (width 0.25) (layer B.Cu) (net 8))
 (segment (start 216.3572 84.0994) (end 216.3572 82.8741) (width 0.25) (layer B.Cu) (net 8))
 (segment (start 216.3572 82.8741) (end 213.638 80.1549) (width 0.25) (layer B.Cu) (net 8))
 (segment (start 213.638 80.1549) (end 213.638 76.466) (width 0.25) (layer B.Cu) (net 8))
 (segment (start 213.638 76.466) (end 213.5354 76.3634) (width 0.25) (layer B.Cu) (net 8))
 (segment (start 213.678 74.295) (end 213.638 74.335) (width 0.25) (layer B.Cu) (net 8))
 (segment (start 213.638 74.335) (end 213.638 74.875) (width 0.25) (layer B.Cu) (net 8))
 (segment (start 213.678 93.345) (end 213.638 93.385) (width 0.25) (layer B.Cu) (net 7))
 (segment (start 213.638 93.385) (end 213.638 93.925) (width 0.25) (layer B.Cu) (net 7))
 (segment (start 213.638 93.925) (end 213.5354 95.4134) (width 0.25) (layer B.Cu) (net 7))
 (segment (start 216.535 104.775) (end 216.535 103.5497) (width 0.25) (layer B.Cu) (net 7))
 (segment (start 216.535 103.5497) (end 213.638 100.6527) (width 0.25) (layer B.Cu) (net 7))
 (segment (start 213.638 100.6527) (end 213.638 95.516) (width 0.25) (layer B.Cu) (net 7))
 (segment (start 213.638 95.516) (end 213.5354 95.4134) (width 0.25) (layer B.Cu) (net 7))
 (segment (start 213.678 112.395) (end 213.638 112.435) (width 0.25) (layer B.Cu) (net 5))
 (segment (start 213.638 112.435) (end 213.638 112.975) (width 0.25) (layer B.Cu) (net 5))
 (segment (start 213.638 112.975) (end 213.5354 114.4634) (width 0.25) (layer B.Cu) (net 5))
 (segment (start 216.535 123.031) (end 216.535 121.8057) (width 0.25) (layer B.Cu) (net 5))
 (segment (start 216.535 121.8057) (end 213.638 118.9087) (width 0.25) (layer B.Cu) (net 5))
 (segment (start 213.638 118.9087) (end 213.638 114.566) (width 0.25) (layer B.Cu) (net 5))
 (segment (start 213.638 114.566) (end 213.5354 114.4634) (width 0.25) (layer B.Cu) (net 5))
 (segment (start 232.728 74.295) (end 232.688 74.335) (width 0.25) (layer B.Cu) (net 4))
 (segment (start 232.688 74.335) (end 232.688 74.875) (width 0.25) (layer B.Cu) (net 4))
 (segment (start 232.688 74.875) (end 232.5854 76.3634) (width 0.25) (layer B.Cu) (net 4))
 (segment (start 235.585 84.9312) (end 235.585 83.7059) (width 0.25) (layer B.Cu) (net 4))
 (segment (start 235.585 83.7059) (end 232.688 80.8089) (width 0.25) (layer B.Cu) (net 4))
 (segment (start 232.688 80.8089) (end 232.688 76.466) (width 0.25) (layer B.Cu) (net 4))
 (segment (start 232.688 76.466) (end 232.5854 76.3634) (width 0.25) (layer B.Cu) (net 4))
 (segment (start 232.728 93.345) (end 232.688 93.385) (width 0.25) (layer B.Cu) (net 3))
 (segment (start 232.688 93.385) (end 232.688 93.925) (width 0.25) (layer B.Cu) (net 3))
 (segment (start 232.688 93.925) (end 232.5854 95.4134) (width 0.25) (layer B.Cu) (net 3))
 (segment (start 235.585 103.981) (end 235.585 102.7557) (width 0.25) (layer B.Cu) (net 3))
 (segment (start 235.585 102.7557) (end 232.688 99.8587) (width 0.25) (layer B.Cu) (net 3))
 (segment (start 232.688 99.8587) (end 232.688 95.516) (width 0.25) (layer B.Cu) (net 3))
 (segment (start 232.688 95.516) (end 232.5854 95.4134) (width 0.25) (layer B.Cu) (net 3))
 (segment (start 232.728 112.395) (end 232.688 112.435) (width 0.25) (layer B.Cu) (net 1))
 (segment (start 232.688 112.435) (end 232.688 112.975) (width 0.25) (layer B.Cu) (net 1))
 (segment (start 232.688 112.975) (end 232.5854 114.4634) (width 0.25) (layer B.Cu) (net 1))
 (segment (start 234.791 123.031) (end 234.791 121.8057) (width 0.25) (layer B.Cu) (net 1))
 (segment (start 234.791 121.8057) (end 232.688 119.7027) (width 0.25) (layer B.Cu) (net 1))
 (segment (start 232.688 119.7027) (end 232.688 114.566) (width 0.25) (layer B.Cu) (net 1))
 (segment (start 232.688 114.566) (end 232.5854 114.4634) (width 0.25) (layer B.Cu) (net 1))
 (segment (start 188.278 95.885) (end 187.2877 96.9887) (width 0.25) (layer F.Cu) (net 10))
 (segment (start 187.2877 96.9887) (end 188.278 97.979) (width 0.25) (layer F.Cu) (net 10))
 (segment (start 188.278 97.979) (end 188.278 112.165) (width 0.25) (layer F.Cu) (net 10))
 (segment (start 188.278 112.165) (end 189.588 113.475) (width 0.25) (layer F.Cu) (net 10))
 (segment (start 189.588 113.475) (end 188.278 114.785) (width 0.25) (layer B.Cu) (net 10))
 (segment (start 188.278 114.785) (end 188.278 114.935) (width 0.25) (layer B.Cu) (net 10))
 (segment (start 189.588 94.425) (end 188.278 95.735) (width 0.25) (layer B.Cu) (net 10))
 (segment (start 188.278 95.735) (end 188.278 95.885) (width 0.25) (layer B.Cu) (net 10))
 (segment (start 189.588 94.425) (end 185.41 90.247) (width 0.25) (layer B.Cu) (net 10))
 (segment (start 185.41 90.247) (end 185.41 82.7646) (width 0.25) (layer B.Cu) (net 10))
 (segment (start 185.41 82.7646) (end 188.2087 79.9659) (width 0.25) (layer B.Cu) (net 10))
 (segment (start 188.2087 79.9659) (end 188.2087 78.8597) (width 0.25) (layer B.Cu) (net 10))
 (segment (start 188.2087 78.8597) (end 187.2877 77.9387) (width 0.25) (layer B.Cu) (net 10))
 (segment (start 188.278 76.835) (end 187.2877 77.9387) (width 0.25) (layer B.Cu) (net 10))
 (segment (start 189.588 75.375) (end 188.278 76.685) (width 0.25) (layer B.Cu) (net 10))
 (segment (start 188.278 76.685) (end 188.278 76.835) (width 0.25) (layer B.Cu) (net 10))
 (segment (start 203.518 88.9) (end 195.113 88.9) (width 0.25) (layer F.Cu) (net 10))
 (segment (start 195.113 88.9) (end 189.588 94.425) (width 0.25) (layer F.Cu) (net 10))
 (segment (start 203.518 86.36) (end 208.638 91.48) (width 0.25) (layer B.Cu) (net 6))
 (segment (start 208.638 91.48) (end 208.638 94.425) (width 0.25) (layer B.Cu) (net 6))
 (segment (start 206.3377 77.9387) (end 205.723 77.9387) (width 0.25) (layer B.Cu) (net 6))
 (segment (start 205.723 77.9387) (end 204.8333 78.8284) (width 0.25) (layer B.Cu) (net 6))
 (segment (start 204.8333 78.8284) (end 204.8333 85.0447) (width 0.25) (layer B.Cu) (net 6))
 (segment (start 204.8333 85.0447) (end 203.518 86.36) (width 0.25) (layer B.Cu) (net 6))
 (segment (start 207.328 95.885) (end 206.3377 96.9887) (width 0.25) (layer B.Cu) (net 6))
 (segment (start 208.638 113.475) (end 208.638 99.289) (width 0.25) (layer B.Cu) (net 6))
 (segment (start 208.638 99.289) (end 206.3377 96.9887) (width 0.25) (layer B.Cu) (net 6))
 (segment (start 208.638 113.475) (end 207.328 114.785) (width 0.25) (layer F.Cu) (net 6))
 (segment (start 207.328 114.785) (end 207.328 114.935) (width 0.25) (layer F.Cu) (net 6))
 (segment (start 207.328 95.885) (end 208.638 94.425) (width 0.25) (layer B.Cu) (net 6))
 (segment (start 207.328 76.835) (end 206.3377 77.9387) (width 0.25) (layer B.Cu) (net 6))
 (segment (start 208.638 75.375) (end 207.328 76.685) (width 0.25) (layer B.Cu) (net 6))
 (segment (start 207.328 76.685) (end 207.328 76.835) (width 0.25) (layer B.Cu) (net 6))
 (segment (start 226.378 76.835) (end 225.3877 77.9387) (width 0.25) (layer F.Cu) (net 2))
 (segment (start 203.518 83.82) (end 205.2322 82.1058) (width 0.25) (layer F.Cu) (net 2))
 (segment (start 205.2322 82.1058) (end 215.4672 82.1058) (width 0.25) (layer F.Cu) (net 2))
 (segment (start 215.4672 82.1058) (end 217.563 80.01) (width 0.25) (layer F.Cu) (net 2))
 (segment (start 217.563 80.01) (end 220.074 80.01) (width 0.25) (layer F.Cu) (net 2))
 (segment (start 220.074 80.01) (end 222.1453 77.9387) (width 0.25) (layer F.Cu) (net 2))
 (segment (start 222.1453 77.9387) (end 225.3877 77.9387) (width 0.25) (layer F.Cu) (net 2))
 (segment (start 227.688 94.425) (end 226.378 95.735) (width 0.25) (layer F.Cu) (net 2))
 (segment (start 226.378 95.735) (end 226.378 95.885) (width 0.25) (layer F.Cu) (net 2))
 (segment (start 226.378 76.835) (end 225.3877 77.9387) (width 0.25) (layer B.Cu) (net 2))
 (segment (start 225.3877 77.9387) (end 227.688 80.239) (width 0.25) (layer B.Cu) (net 2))
 (segment (start 227.688 80.239) (end 227.688 94.425) (width 0.25) (layer B.Cu) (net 2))
 (segment (start 227.688 75.375) (end 226.378 76.685) (width 0.25) (layer B.Cu) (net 2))
 (segment (start 226.378 76.685) (end 226.378 76.835) (width 0.25) (layer B.Cu) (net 2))
 (segment (start 227.033 113.475) (end 227.033 98.634) (width 0.25) (layer B.Cu) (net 2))
 (segment (start 227.033 98.634) (end 225.3877 96.9887) (width 0.25) (layer B.Cu) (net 2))
 (segment (start 226.378 114.935) (end 226.378 114.13) (width 0.25) (layer B.Cu) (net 2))
 (segment (start 226.378 114.13) (end 227.033 113.475) (width 0.25) (layer B.Cu) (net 2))
 (segment (start 227.688 113.475) (end 227.033 113.475) (width 0.25) (layer B.Cu) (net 2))
 (segment (start 226.378 95.885) (end 225.3877 96.9887) (width 0.25) (layer B.Cu) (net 2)))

